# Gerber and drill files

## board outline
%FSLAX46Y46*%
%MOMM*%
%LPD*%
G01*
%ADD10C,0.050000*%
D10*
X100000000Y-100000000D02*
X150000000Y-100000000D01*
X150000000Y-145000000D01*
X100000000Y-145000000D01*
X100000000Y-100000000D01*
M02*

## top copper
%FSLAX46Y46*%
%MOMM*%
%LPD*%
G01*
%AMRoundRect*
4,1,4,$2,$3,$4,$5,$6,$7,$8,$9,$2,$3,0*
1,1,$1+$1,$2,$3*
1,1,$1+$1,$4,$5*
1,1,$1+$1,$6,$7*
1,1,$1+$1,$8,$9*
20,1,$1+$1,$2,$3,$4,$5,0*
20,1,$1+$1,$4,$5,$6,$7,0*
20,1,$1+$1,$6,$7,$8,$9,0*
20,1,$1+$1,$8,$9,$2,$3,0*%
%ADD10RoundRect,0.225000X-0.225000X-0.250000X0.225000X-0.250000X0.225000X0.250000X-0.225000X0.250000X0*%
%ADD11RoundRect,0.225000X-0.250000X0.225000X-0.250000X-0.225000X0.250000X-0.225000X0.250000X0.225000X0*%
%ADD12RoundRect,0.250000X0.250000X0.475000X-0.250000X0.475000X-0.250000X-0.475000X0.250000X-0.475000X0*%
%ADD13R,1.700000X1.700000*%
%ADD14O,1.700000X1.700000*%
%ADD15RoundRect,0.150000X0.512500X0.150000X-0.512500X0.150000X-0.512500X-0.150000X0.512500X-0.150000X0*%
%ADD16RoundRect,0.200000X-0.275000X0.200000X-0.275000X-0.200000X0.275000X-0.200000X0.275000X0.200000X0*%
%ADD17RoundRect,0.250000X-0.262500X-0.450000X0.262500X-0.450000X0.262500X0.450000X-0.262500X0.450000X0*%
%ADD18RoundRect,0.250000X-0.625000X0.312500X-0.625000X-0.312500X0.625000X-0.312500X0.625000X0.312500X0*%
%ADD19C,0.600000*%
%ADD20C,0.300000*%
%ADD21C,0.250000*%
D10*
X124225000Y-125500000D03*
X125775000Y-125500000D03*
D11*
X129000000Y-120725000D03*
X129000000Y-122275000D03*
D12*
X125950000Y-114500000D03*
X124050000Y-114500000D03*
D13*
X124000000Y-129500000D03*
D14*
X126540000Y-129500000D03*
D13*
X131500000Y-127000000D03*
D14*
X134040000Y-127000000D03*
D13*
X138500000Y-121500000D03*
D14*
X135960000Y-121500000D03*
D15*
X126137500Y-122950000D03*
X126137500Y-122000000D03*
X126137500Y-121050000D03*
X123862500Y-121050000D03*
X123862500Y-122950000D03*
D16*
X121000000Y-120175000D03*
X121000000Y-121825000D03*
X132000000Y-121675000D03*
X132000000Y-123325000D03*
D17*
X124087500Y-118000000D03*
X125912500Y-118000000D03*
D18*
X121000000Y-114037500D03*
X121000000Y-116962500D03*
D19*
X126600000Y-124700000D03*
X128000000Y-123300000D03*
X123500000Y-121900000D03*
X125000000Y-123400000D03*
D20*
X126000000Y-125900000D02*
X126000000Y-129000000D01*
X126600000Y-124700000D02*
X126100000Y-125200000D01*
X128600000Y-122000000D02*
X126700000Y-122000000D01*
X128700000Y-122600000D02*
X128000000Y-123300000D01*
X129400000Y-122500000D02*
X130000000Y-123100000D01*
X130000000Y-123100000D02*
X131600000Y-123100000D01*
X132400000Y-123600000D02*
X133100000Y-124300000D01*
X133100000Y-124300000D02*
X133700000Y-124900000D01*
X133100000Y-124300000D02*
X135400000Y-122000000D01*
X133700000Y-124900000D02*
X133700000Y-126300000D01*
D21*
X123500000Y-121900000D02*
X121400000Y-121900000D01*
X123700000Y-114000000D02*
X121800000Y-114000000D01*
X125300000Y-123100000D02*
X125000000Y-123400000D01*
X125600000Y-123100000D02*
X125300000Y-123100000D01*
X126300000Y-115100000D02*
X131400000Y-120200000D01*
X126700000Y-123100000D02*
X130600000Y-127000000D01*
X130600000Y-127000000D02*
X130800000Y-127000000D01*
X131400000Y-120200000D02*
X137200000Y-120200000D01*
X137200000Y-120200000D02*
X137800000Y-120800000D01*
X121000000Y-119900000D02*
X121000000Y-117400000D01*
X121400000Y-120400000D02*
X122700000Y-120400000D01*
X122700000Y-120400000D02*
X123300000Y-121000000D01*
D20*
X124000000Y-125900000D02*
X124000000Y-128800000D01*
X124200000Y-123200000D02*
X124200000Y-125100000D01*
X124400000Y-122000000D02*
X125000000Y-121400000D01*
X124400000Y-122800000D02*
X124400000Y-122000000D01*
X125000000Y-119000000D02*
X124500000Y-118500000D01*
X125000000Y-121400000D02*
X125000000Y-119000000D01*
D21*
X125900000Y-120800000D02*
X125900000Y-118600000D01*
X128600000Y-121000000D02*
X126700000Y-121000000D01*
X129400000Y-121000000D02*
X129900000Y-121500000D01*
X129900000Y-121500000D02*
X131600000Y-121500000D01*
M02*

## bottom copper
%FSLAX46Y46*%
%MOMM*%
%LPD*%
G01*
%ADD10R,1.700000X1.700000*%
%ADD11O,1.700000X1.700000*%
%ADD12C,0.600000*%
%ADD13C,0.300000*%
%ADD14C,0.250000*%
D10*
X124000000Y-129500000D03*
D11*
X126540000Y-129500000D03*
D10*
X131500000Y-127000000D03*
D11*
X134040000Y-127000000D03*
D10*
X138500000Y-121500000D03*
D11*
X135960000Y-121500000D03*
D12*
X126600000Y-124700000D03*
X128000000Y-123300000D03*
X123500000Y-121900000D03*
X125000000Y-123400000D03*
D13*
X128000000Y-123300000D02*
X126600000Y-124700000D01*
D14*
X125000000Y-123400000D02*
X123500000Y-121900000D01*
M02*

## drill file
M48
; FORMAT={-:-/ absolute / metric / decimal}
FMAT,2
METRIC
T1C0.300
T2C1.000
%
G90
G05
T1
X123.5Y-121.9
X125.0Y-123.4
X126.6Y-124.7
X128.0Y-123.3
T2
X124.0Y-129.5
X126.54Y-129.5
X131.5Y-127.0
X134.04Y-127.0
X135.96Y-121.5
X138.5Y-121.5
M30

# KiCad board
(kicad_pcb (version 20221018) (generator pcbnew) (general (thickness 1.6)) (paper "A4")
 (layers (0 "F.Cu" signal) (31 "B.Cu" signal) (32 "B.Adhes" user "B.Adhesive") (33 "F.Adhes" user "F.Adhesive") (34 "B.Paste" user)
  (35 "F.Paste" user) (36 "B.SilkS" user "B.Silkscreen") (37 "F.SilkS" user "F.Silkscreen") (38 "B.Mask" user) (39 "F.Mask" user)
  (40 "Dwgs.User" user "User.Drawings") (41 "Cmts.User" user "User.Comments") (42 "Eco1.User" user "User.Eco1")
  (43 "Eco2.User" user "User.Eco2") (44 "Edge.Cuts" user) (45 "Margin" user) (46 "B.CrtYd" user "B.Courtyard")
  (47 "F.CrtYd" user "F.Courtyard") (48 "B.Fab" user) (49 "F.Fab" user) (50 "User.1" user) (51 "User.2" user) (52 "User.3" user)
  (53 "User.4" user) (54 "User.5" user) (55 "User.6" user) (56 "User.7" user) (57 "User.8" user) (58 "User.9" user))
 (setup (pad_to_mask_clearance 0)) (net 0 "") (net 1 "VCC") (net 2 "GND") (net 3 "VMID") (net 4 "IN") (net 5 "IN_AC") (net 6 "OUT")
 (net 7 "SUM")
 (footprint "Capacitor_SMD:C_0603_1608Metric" (layer "F.Cu") (at 125 125.5)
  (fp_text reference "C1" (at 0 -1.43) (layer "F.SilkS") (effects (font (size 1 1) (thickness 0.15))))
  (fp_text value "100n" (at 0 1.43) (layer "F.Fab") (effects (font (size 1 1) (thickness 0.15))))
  (pad "1" smd roundrect (at -0.775 0) (size 0.9 0.95) (layers "F.Cu" "F.Paste" "F.Mask") (roundrect_rratio 0.25) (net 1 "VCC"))
  (pad "2" smd roundrect (at 0.775 0) (size 0.9 0.95) (layers "F.Cu" "F.Paste" "F.Mask") (roundrect_rratio 0.25) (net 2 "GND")))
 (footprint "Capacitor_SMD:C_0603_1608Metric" (layer "F.Cu") (at 129 121.5 -90)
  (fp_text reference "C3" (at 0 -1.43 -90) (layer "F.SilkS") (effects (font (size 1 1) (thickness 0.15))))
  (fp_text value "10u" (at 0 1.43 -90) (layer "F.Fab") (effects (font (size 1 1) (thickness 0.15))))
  (pad "1" smd roundrect (at -0.775 0 270) (size 0.9 0.95) (layers "F.Cu" "F.Paste" "F.Mask") (roundrect_rratio 0.25) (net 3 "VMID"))
  (pad "2" smd roundrect (at 0.775 0 270) (size 0.9 0.95) (layers "F.Cu" "F.Paste" "F.Mask") (roundrect_rratio 0.25) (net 2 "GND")))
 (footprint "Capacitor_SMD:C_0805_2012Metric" (layer "F.Cu") (at 125 114.5 180)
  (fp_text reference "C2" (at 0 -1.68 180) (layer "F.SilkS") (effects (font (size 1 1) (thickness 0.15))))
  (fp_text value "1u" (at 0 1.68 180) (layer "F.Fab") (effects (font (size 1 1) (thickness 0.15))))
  (pad "1" smd roundrect (at -0.95 0 180) (size 1 1.45) (layers "F.Cu" "F.Paste" "F.Mask") (roundrect_rratio 0.25) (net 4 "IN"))
  (pad "2" smd roundrect (at 0.95 0 180) (size 1 1.45) (layers "F.Cu" "F.Paste" "F.Mask") (roundrect_rratio 0.25) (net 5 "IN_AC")))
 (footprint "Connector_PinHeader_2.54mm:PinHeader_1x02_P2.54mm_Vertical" (layer "F.Cu") (at 124 129.5 90)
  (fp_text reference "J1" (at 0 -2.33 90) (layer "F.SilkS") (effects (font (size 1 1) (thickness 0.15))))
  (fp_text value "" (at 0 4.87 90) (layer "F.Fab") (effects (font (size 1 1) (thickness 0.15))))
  (pad "1" thru_hole rect (at 0 0 90) (size 1.7 1.7) (drill 1) (layers "*.Cu" "*.Mask") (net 1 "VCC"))
  (pad "2" thru_hole oval (at 0 2.54 90) (size 1.7 1.7) (drill 1) (layers "*.Cu" "*.Mask") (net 2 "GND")))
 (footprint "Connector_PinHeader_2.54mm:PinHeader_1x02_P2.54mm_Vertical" (layer "F.Cu") (at 131.5 127 90)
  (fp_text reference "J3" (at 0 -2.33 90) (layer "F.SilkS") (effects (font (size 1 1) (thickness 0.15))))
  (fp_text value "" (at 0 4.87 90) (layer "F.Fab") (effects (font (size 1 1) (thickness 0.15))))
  (pad "1" thru_hole rect (at 0 0 90) (size 1.7 1.7) (drill 1) (layers "*.Cu" "*.Mask") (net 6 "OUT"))
  (pad "2" thru_hole oval (at 0 2.54 90) (size 1.7 1.7) (drill 1) (layers "*.Cu" "*.Mask") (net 2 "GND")))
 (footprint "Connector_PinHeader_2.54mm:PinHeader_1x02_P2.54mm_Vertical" (layer "F.Cu") (at 138.5 121.5 -90)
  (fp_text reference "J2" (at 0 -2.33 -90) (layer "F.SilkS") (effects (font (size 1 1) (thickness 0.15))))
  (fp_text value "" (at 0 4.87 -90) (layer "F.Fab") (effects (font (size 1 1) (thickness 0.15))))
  (pad "1" thru_hole rect (at 0 0 270) (size 1.7 1.7) (drill 1) (layers "*.Cu" "*.Mask") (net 4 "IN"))
  (pad "2" thru_hole oval (at 0 2.54 270) (size 1.7 1.7) (drill 1) (layers "*.Cu" "*.Mask") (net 2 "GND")))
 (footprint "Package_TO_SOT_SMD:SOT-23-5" (layer "F.Cu") (at 125 122 180)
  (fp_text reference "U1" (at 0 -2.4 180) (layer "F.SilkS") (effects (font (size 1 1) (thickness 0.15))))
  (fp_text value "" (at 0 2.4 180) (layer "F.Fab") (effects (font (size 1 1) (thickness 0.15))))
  (pad "1" smd roundrect (at -1.1375 -0.95 180) (size 1.325 0.6) (layers "F.Cu" "F.Paste" "F.Mask") (roundrect_rratio 0.25) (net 6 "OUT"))
  (pad "2" smd roundrect (at -1.1375 0 180) (size 1.325 0.6) (layers "F.Cu" "F.Paste" "F.Mask") (roundrect_rratio 0.25) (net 2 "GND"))
  (pad "3" smd roundrect (at -1.1375 0.95 180) (size 1.325 0.6) (layers "F.Cu" "F.Paste" "F.Mask") (roundrect_rratio 0.25) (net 3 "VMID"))
  (pad "4" smd roundrect (at 1.1375 0.95 180) (size 1.325 0.6) (layers "F.Cu" "F.Paste" "F.Mask") (roundrect_rratio 0.25) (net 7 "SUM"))
  (pad "5" smd roundrect (at 1.1375 -0.95 180) (size 1.325 0.6) (layers "F.Cu" "F.Paste" "F.Mask") (roundrect_rratio 0.25) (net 1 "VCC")))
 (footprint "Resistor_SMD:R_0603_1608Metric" (layer "F.Cu") (at 121 121 -90)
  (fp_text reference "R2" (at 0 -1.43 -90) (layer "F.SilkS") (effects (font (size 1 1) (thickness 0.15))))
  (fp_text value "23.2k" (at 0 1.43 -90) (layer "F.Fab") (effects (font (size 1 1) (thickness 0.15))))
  (pad "1" smd roundrect (at -0.825 0 270) (size 0.8 0.95) (layers "F.Cu" "F.Paste" "F.Mask") (roundrect_rratio 0.25) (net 7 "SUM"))
  (pad "2" smd roundrect (at 0.825 0 270) (size 0.8 0.95) (layers "F.Cu" "F.Paste" "F.Mask") (roundrect_rratio 0.25) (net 6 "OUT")))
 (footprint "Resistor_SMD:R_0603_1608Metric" (layer "F.Cu") (at 132 122.5 -90)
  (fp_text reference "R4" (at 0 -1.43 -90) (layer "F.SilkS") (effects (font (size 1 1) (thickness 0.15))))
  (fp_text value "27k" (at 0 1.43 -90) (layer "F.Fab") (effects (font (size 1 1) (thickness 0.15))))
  (pad "1" smd roundrect (at -0.825 0 270) (size 0.8 0.95) (layers "F.Cu" "F.Paste" "F.Mask") (roundrect_rratio 0.25) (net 3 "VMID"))
  (pad "2" smd roundrect (at 0.825 0 270) (size 0.8 0.95) (layers "F.Cu" "F.Paste" "F.Mask") (roundrect_rratio 0.25) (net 2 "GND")))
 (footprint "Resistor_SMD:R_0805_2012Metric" (layer "F.Cu") (at 125 118)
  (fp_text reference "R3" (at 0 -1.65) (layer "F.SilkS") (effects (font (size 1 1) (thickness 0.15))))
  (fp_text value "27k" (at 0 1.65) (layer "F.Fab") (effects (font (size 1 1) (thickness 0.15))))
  (pad "1" smd roundrect (at -0.9125 0) (size 1.025 1.4) (layers "F.Cu" "F.Paste" "F.Mask") (roundrect_rratio 0.243902) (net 1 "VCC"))
  (pad "2" smd roundrect (at 0.9125 0) (size 1.025 1.4) (layers "F.Cu" "F.Paste" "F.Mask") (roundrect_rratio 0.243902) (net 3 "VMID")))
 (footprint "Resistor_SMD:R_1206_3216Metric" (layer "F.Cu") (at 121 115.5 -90)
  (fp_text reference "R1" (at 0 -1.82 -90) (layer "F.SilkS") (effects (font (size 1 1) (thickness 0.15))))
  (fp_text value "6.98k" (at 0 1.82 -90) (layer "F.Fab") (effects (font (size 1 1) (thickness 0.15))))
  (pad "1" smd roundrect (at -1.4625 0 270) (size 1.125 1.75) (layers "F.Cu" "F.Paste" "F.Mask") (roundrect_rratio 0.222222) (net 5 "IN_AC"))
  (pad "2" smd roundrect (at 1.4625 0 270) (size 1.125 1.75) (layers "F.Cu" "F.Paste" "F.Mask") (roundrect_rratio 0.222222) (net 7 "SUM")))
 (gr_rect (start 100 100) (end 150 145) (stroke (width 0.05) (type default)) (fill none) (layer "Edge.Cuts"))
 (segment (start 126 125.9) (end 126 129) (width 0.3) (layer "F.Cu") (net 2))
 (segment (start 126.6 124.7) (end 126.1 125.2) (width 0.3) (layer "F.Cu") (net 2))
 (segment (start 128.6 122) (end 126.7 122) (width 0.3) (layer "F.Cu") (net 2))
 (segment (start 128.7 122.6) (end 128 123.3) (width 0.3) (layer "F.Cu") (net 2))
 (segment (start 129.4 122.5) (end 130 123.1) (width 0.3) (layer "F.Cu") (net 2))
 (segment (start 130 123.1) (end 131.6 123.1) (width 0.3) (layer "F.Cu") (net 2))
 (segment (start 132.4 123.6) (end 133.1 124.3) (width 0.3) (layer "F.Cu") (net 2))
 (segment (start 133.1 124.3) (end 133.7 124.9) (width 0.3) (layer "F.Cu") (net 2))
 (segment (start 133.1 124.3) (end 135.4 122) (width 0.3) (layer "F.Cu") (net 2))
 (segment (start 133.7 124.9) (end 133.7 126.3) (width 0.3) (layer "F.Cu") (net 2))
 (via (at 126.6 124.7) (size 0.6) (drill 0.3) (layers "F.Cu" "B.Cu") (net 2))
 (via (at 128 123.3) (size 0.6) (drill 0.3) (layers "F.Cu" "B.Cu") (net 2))
 (segment (start 123.5 121.9) (end 121.4 121.9) (width 0.25) (layer "F.Cu") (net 6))
 (segment (start 123.7 114) (end 121.8 114) (width 0.25) (layer "F.Cu") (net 5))
 (segment (start 125.3 123.1) (end 125 123.4) (width 0.25) (layer "F.Cu") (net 6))
 (segment (start 125.6 123.1) (end 125.3 123.1) (width 0.25) (layer "F.Cu") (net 6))
 (segment (start 126.3 115.1) (end 131.4 120.2) (width 0.25) (layer "F.Cu") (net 4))
 (segment (start 126.7 123.1) (end 130.6 127) (width 0.25) (layer "F.Cu") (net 6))
 (segment (start 128 123.3) (end 126.6 124.7) (width 0.3) (layer "B.Cu") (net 2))
 (segment (start 130.6 127) (end 130.8 127) (width 0.25) (layer "F.Cu") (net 6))
 (segment (start 131.4 120.2) (end 137.2 120.2) (width 0.25) (layer "F.Cu") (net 4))
 (segment (start 137.2 120.2) (end 137.8 120.8) (width 0.25) (layer "F.Cu") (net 4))
 (via (at 123.5 121.9) (size 0.6) (drill 0.3) (layers "F.Cu" "B.Cu") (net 6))
 (via (at 125 123.4) (size 0.6) (drill 0.3) (layers "F.Cu" "B.Cu") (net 6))
 (segment (start 121 119.9) (end 121 117.4) (width 0.25) (layer "F.Cu") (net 7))
 (segment (start 121.4 120.4) (end 122.7 120.4) (width 0.25) (layer "F.Cu") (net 7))
 (segment (start 122.7 120.4) (end 123.3 121) (width 0.25) (layer "F.Cu") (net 7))
 (segment (start 124 125.9) (end 124 128.8) (width 0.3) (layer "F.Cu") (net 1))
 (segment (start 124.2 123.2) (end 124.2 125.1) (width 0.3) (layer "F.Cu") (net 1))
 (segment (start 124.4 122) (end 125 121.4) (width 0.3) (layer "F.Cu") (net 1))
 (segment (start 124.4 122.8) (end 124.4 122) (width 0.3) (layer "F.Cu") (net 1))
 (segment (start 125 119) (end 124.5 118.5) (width 0.3) (layer "F.Cu") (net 1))
 (segment (start 125 121.4) (end 125 119) (width 0.3) (layer "F.Cu") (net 1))
 (segment (start 125 123.4) (end 123.5 121.9) (width 0.25) (layer "B.Cu") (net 6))
 (segment (start 125.9 120.8) (end 125.9 118.6) (width 0.25) (layer "F.Cu") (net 3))
 (segment (start 128.6 121) (end 126.7 121) (width 0.25) (layer "F.Cu") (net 3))
 (segment (start 129.4 121) (end 129.9 121.5) (width 0.25) (layer "F.Cu") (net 3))
 (segment (start 129.9 121.5) (end 131.6 121.5) (width 0.25) (layer "F.Cu") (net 3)))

